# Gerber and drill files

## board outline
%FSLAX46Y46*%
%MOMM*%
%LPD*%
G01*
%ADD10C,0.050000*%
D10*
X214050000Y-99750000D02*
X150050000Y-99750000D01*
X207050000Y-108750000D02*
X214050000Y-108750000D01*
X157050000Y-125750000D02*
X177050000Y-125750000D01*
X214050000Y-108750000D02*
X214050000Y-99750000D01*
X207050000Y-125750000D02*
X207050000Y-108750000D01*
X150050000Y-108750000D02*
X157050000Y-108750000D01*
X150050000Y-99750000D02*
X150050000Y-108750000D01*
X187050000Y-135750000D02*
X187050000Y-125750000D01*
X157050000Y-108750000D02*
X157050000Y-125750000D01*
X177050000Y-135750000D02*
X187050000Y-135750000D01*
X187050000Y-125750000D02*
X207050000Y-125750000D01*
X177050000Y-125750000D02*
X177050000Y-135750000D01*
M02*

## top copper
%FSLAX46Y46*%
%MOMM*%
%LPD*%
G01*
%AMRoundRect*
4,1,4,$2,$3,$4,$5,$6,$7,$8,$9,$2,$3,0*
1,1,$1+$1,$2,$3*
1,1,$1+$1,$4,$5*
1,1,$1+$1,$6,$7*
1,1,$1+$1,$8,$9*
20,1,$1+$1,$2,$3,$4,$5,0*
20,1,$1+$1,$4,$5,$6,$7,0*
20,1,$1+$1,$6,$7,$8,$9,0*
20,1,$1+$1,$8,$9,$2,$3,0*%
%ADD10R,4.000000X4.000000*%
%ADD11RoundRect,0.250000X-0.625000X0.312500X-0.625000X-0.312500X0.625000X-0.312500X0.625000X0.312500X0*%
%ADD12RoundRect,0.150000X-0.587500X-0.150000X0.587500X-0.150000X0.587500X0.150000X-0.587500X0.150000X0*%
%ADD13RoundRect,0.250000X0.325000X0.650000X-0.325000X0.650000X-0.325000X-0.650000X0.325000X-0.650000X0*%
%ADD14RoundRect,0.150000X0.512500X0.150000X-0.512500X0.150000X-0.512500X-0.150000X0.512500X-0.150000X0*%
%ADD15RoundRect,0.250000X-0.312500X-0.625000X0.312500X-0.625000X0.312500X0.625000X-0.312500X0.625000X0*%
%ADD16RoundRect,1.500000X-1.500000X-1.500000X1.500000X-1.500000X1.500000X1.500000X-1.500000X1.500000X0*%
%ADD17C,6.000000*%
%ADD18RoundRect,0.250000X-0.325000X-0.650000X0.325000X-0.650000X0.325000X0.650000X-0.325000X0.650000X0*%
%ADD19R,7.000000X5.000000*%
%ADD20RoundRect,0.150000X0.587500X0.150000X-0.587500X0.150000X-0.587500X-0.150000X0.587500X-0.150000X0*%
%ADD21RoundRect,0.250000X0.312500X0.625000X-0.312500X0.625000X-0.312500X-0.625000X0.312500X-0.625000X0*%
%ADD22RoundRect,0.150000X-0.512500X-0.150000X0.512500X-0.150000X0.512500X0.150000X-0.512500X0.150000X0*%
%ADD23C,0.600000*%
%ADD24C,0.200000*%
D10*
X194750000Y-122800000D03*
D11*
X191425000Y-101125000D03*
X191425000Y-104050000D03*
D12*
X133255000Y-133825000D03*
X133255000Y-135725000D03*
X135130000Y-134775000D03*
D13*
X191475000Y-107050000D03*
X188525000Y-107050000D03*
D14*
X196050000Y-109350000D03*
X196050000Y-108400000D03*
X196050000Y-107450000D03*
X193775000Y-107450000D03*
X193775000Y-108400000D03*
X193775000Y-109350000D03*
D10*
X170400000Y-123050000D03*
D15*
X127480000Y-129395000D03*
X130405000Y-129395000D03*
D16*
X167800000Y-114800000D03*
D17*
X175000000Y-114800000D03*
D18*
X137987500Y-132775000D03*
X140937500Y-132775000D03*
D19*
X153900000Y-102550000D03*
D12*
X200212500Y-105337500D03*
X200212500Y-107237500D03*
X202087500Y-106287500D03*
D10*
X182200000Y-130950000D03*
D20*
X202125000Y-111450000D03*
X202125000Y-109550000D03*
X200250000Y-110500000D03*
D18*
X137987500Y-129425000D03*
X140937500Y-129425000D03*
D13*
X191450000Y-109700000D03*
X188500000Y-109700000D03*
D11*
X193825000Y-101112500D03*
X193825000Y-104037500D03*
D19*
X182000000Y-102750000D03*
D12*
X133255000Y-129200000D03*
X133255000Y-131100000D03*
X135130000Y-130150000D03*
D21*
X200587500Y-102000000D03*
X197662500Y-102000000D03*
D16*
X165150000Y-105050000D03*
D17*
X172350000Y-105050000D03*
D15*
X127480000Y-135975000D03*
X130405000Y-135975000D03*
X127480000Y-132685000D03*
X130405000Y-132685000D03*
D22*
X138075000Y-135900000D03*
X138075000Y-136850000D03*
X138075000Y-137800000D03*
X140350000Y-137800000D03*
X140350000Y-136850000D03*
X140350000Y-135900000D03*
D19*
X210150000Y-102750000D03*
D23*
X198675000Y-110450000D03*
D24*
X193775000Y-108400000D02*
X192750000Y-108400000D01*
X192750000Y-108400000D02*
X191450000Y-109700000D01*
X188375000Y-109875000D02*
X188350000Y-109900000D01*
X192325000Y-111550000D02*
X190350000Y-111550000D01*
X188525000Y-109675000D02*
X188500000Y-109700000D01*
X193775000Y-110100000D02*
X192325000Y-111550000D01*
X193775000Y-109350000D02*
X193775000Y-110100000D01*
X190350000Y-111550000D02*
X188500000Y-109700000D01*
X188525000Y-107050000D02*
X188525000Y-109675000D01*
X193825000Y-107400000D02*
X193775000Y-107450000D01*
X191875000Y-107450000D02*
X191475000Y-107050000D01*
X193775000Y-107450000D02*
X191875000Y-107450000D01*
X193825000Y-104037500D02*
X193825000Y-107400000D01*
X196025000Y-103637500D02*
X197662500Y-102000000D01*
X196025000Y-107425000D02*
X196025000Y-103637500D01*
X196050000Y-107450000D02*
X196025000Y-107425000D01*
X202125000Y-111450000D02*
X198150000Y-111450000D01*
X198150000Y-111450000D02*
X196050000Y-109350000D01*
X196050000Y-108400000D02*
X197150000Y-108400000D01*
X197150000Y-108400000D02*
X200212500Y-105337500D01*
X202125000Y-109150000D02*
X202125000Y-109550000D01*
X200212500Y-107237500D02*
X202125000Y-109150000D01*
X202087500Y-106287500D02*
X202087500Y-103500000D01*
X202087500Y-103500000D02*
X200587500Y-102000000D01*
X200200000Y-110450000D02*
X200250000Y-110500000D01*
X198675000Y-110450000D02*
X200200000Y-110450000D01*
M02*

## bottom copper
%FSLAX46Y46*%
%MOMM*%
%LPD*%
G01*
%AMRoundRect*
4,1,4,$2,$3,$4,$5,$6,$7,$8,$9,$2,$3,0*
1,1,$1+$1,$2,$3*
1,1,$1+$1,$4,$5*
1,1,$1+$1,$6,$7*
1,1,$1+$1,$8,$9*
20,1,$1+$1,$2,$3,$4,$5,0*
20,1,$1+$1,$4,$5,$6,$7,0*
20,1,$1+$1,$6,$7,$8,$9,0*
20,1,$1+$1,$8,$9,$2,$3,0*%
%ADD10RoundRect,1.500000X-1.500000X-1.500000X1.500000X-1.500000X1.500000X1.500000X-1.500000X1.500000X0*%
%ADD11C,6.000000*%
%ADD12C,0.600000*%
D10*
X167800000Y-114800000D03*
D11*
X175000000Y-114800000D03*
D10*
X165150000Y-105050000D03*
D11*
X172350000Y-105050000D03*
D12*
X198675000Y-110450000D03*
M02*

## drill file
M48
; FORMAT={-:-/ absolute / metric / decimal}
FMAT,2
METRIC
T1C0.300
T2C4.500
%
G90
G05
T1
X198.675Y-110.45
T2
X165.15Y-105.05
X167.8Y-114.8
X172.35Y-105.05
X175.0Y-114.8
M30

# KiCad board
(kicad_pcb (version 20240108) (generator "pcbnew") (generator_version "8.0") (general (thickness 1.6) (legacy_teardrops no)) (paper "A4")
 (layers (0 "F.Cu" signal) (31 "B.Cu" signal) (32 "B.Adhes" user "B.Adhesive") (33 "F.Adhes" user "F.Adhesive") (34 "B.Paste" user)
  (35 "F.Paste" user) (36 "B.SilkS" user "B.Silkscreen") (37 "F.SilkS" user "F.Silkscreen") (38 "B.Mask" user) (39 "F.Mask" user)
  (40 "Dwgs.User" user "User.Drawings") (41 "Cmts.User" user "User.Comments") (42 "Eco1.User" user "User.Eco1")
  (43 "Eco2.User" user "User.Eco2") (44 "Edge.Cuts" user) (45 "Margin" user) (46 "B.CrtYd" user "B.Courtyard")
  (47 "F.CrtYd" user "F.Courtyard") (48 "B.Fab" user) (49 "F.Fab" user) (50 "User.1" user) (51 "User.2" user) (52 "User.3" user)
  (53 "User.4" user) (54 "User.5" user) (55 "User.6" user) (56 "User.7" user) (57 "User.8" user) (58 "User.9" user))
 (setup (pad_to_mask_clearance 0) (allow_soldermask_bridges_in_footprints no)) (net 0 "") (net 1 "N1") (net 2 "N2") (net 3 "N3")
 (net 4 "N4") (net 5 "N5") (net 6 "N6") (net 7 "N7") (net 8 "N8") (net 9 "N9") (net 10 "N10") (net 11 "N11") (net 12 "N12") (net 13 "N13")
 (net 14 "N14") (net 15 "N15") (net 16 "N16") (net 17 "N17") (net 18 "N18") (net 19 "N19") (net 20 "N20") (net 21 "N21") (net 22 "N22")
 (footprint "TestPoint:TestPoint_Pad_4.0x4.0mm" (layer "F.Cu") (at 194.75 122.8)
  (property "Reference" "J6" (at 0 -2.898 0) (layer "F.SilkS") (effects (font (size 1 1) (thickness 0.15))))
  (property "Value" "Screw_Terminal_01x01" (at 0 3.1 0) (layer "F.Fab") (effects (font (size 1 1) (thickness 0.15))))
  (pad "1" smd rect (at 0 0) (size 4 4) (layers "F.Cu" "F.Mask") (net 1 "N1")))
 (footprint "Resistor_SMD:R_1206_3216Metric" (layer "F.Cu") (at 191.425 102.5875 -90)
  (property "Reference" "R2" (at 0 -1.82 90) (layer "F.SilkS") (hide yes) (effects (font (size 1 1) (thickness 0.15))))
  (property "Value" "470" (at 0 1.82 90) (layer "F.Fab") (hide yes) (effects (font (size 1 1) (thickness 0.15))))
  (pad "1" smd roundrect (at -1.4625 0 270) (size 1.125 1.75) (layers "F.Cu" "F.Paste" "F.Mask") (roundrect_rratio 0.222222) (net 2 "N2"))
  (pad "2" smd roundrect (at 1.4625 0 270) (size 1.125 1.75) (layers "F.Cu" "F.Paste" "F.Mask") (roundrect_rratio 0.222222) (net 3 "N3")))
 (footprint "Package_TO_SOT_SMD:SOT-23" (layer "F.Cu") (at 134.1925 134.775)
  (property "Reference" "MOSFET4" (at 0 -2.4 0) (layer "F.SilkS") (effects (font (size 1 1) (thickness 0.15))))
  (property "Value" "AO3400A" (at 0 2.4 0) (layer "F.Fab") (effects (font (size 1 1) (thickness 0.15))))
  (pad "1" smd roundrect (at -0.9375 -0.95) (size 1.475 0.6) (layers "F.Cu" "F.Paste" "F.Mask") (roundrect_rratio 0.25) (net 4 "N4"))
  (pad "2" smd roundrect (at -0.9375 0.95) (size 1.475 0.6) (layers "F.Cu" "F.Paste" "F.Mask") (roundrect_rratio 0.25) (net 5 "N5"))
  (pad "3" smd roundrect (at 0.9375 0) (size 1.475 0.6) (layers "F.Cu" "F.Paste" "F.Mask") (roundrect_rratio 0.25) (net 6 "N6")))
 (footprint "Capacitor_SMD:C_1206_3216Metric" (layer "F.Cu") (at 190 107.05 180)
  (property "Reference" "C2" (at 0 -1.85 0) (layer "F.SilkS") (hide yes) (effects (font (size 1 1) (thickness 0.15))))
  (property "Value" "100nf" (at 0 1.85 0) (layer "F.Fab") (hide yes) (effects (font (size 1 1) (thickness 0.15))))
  (pad "1" smd roundrect (at -1.475 0 180) (size 1.15 1.8) (layers "F.Cu" "F.Paste" "F.Mask") (roundrect_rratio 0.217391) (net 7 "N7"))
  (pad "2" smd roundrect (at 1.475 0 180) (size 1.15 1.8) (layers "F.Cu" "F.Paste" "F.Mask") (roundrect_rratio 0.217391) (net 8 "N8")))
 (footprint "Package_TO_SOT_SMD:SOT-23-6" (layer "F.Cu") (at 194.9125 108.4 180)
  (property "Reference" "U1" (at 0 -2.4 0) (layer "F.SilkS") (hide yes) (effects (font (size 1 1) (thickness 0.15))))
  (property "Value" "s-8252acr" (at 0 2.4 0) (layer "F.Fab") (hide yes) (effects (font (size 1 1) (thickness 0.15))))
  (pad "1" smd roundrect (at -1.1375 -0.95 180) (size 1.325 0.6) (layers "F.Cu" "F.Paste" "F.Mask") (roundrect_rratio 0.25) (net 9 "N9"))
  (pad "2" smd roundrect (at -1.1375 0 180) (size 1.325 0.6) (layers "F.Cu" "F.Paste" "F.Mask") (roundrect_rratio 0.25) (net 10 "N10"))
  (pad "3" smd roundrect (at -1.1375 0.95 180) (size 1.325 0.6) (layers "F.Cu" "F.Paste" "F.Mask") (roundrect_rratio 0.25) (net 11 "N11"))
  (pad "4" smd roundrect (at 1.1375 0.95 180) (size 1.325 0.6) (layers "F.Cu" "F.Paste" "F.Mask") (roundrect_rratio 0.25) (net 7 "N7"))
  (pad "5" smd roundrect (at 1.1375 0 180) (size 1.325 0.6) (layers "F.Cu" "F.Paste" "F.Mask") (roundrect_rratio 0.25) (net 3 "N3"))
  (pad "6" smd roundrect (at 1.1375 -0.95 180) (size 1.325 0.6) (layers "F.Cu" "F.Paste" "F.Mask") (roundrect_rratio 0.25) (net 8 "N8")))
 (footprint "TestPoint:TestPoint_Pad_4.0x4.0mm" (layer "F.Cu") (at 170.4 123.05)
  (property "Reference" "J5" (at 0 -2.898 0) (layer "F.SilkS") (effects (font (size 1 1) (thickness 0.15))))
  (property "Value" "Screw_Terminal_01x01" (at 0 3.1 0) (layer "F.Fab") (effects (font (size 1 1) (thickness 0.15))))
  (pad "1" smd rect (at 0 0) (size 4 4) (layers "F.Cu" "F.Mask") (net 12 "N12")))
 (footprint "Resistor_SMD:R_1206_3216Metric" (layer "F.Cu") (at 128.9425 129.395)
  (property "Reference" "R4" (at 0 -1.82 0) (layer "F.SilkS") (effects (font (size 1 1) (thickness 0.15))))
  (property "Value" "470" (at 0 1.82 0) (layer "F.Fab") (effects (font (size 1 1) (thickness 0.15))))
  (pad "1" smd roundrect (at -1.4625 0) (size 1.125 1.75) (layers "F.Cu" "F.Paste" "F.Mask") (roundrect_rratio 0.222222) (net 12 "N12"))
  (pad "2" smd roundrect (at 1.4625 0) (size 1.125 1.75) (layers "F.Cu" "F.Paste" "F.Mask") (roundrect_rratio 0.222222) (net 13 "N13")))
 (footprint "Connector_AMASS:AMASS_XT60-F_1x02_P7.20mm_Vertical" (layer "F.Cu") (at 167.8 114.8)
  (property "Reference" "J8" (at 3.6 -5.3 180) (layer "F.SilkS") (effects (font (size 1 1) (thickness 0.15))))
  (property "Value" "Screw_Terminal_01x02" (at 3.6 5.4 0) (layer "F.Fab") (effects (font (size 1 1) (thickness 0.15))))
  (pad "1" thru_hole roundrect (at 0 0) (size 6 6) (drill 4.5) (layers "*.Cu" "*.Mask") (remove_unused_layers no) (roundrect_rratio 0.25)
   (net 12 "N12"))
  (pad "2" thru_hole circle (at 7.2 0) (size 6 6) (drill 4.5) (layers "*.Cu" "*.Mask") (remove_unused_layers no) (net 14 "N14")))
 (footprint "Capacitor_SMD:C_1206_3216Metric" (layer "F.Cu") (at 139.4625 132.775)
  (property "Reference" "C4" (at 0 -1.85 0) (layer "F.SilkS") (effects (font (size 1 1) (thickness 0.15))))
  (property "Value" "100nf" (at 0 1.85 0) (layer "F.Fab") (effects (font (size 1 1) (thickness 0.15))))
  (pad "1" smd roundrect (at -1.475 0) (size 1.15 1.8) (layers "F.Cu" "F.Paste" "F.Mask") (roundrect_rratio 0.217391) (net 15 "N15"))
  (pad "2" smd roundrect (at 1.475 0) (size 1.15 1.8) (layers "F.Cu" "F.Paste" "F.Mask") (roundrect_rratio 0.217391) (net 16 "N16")))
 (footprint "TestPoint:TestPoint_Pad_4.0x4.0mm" (layer "F.Cu") (at 153.9 102.55)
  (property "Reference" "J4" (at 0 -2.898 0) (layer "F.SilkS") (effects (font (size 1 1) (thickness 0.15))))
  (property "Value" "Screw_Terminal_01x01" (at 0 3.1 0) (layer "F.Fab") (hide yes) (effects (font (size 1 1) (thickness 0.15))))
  (pad "1" smd rect (at 0 0) (size 7 5) (layers "F.Cu" "F.Mask") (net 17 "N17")))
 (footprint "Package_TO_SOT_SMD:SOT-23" (layer "F.Cu") (at 201.15 106.2875)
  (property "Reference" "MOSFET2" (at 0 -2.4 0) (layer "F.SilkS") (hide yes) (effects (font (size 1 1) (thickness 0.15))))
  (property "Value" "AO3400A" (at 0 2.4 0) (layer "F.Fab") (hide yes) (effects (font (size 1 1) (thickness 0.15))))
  (pad "1" smd roundrect (at -0.9375 -0.95) (size 1.475 0.6) (layers "F.Cu" "F.Paste" "F.Mask") (roundrect_rratio 0.25) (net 10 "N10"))
  (pad "2" smd roundrect (at -0.9375 0.95) (size 1.475 0.6) (layers "F.Cu" "F.Paste" "F.Mask") (roundrect_rratio 0.25) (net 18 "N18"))
  (pad "3" smd roundrect (at 0.9375 0) (size 1.475 0.6) (layers "F.Cu" "F.Paste" "F.Mask") (roundrect_rratio 0.25) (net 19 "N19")))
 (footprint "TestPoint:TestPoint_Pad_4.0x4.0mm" (layer "F.Cu") (at 182.2 130.95)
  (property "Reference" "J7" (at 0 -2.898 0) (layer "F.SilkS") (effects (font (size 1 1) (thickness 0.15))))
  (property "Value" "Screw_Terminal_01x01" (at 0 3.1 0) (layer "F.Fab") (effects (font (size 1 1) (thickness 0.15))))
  (pad "1" smd rect (at 0 0) (size 4 4) (layers "F.Cu" "F.Mask") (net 6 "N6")))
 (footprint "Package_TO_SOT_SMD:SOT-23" (layer "F.Cu") (at 201.1875 110.5 180)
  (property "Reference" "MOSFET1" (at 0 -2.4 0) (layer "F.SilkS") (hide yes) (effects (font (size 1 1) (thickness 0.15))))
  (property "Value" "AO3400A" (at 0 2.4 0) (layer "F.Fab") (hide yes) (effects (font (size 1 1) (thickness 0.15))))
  (pad "1" smd roundrect (at -0.9375 -0.95 180) (size 1.475 0.6) (layers "F.Cu" "F.Paste" "F.Mask") (roundrect_rratio 0.25) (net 9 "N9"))
  (pad "2" smd roundrect (at -0.9375 0.95 180) (size 1.475 0.6) (layers "F.Cu" "F.Paste" "F.Mask") (roundrect_rratio 0.25) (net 18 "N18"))
  (pad "3" smd roundrect (at 0.9375 0 180) (size 1.475 0.6) (layers "F.Cu" "F.Paste" "F.Mask") (roundrect_rratio 0.25) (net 17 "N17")))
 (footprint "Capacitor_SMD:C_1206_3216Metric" (layer "F.Cu") (at 139.4625 129.425)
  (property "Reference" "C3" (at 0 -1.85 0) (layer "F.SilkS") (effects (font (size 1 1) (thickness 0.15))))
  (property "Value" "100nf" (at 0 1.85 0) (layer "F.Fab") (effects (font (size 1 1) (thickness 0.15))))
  (pad "1" smd roundrect (at -1.475 0) (size 1.15 1.8) (layers "F.Cu" "F.Paste" "F.Mask") (roundrect_rratio 0.217391) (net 13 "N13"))
  (pad "2" smd roundrect (at 1.475 0) (size 1.15 1.8) (layers "F.Cu" "F.Paste" "F.Mask") (roundrect_rratio 0.217391) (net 16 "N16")))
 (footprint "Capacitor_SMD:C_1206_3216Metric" (layer "F.Cu") (at 189.975 109.7 180)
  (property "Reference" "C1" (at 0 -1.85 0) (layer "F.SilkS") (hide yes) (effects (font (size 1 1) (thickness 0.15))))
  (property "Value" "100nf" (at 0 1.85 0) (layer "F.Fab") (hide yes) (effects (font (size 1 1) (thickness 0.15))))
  (pad "1" smd roundrect (at -1.475 0 180) (size 1.15 1.8) (layers "F.Cu" "F.Paste" "F.Mask") (roundrect_rratio 0.217391) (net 3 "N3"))
  (pad "2" smd roundrect (at 1.475 0 180) (size 1.15 1.8) (layers "F.Cu" "F.Paste" "F.Mask") (roundrect_rratio 0.217391) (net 8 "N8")))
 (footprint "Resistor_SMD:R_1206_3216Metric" (layer "F.Cu") (at 193.825 102.575 -90)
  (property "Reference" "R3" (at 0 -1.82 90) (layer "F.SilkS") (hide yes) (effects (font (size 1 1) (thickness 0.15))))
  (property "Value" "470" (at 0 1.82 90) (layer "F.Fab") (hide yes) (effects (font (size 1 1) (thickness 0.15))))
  (pad "1" smd roundrect (at -1.4625 0 270) (size 1.125 1.75) (layers "F.Cu" "F.Paste" "F.Mask") (roundrect_rratio 0.222222) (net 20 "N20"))
  (pad "2" smd roundrect (at 1.4625 0 270) (size 1.125 1.75) (layers "F.Cu" "F.Paste" "F.Mask") (roundrect_rratio 0.222222) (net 7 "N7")))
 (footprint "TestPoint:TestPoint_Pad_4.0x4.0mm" (layer "F.Cu") (at 182 102.75)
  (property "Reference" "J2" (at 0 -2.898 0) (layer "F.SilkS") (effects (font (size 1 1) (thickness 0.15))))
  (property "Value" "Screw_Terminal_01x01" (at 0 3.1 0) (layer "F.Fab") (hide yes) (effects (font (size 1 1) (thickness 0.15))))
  (pad "1" smd rect (at 0 0) (size 7 5) (layers "F.Cu" "F.Mask") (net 20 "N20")))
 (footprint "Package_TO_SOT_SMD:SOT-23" (layer "F.Cu") (at 134.1925 130.15)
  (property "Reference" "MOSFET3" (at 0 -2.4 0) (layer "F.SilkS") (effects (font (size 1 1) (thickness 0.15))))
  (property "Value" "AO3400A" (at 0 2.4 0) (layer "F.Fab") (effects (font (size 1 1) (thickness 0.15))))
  (pad "1" smd roundrect (at -0.9375 -0.95) (size 1.475 0.6) (layers "F.Cu" "F.Paste" "F.Mask") (roundrect_rratio 0.25) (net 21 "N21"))
  (pad "2" smd roundrect (at -0.9375 0.95) (size 1.475 0.6) (layers "F.Cu" "F.Paste" "F.Mask") (roundrect_rratio 0.25) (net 5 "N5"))
  (pad "3" smd roundrect (at 0.9375 0) (size 1.475 0.6) (layers "F.Cu" "F.Paste" "F.Mask") (roundrect_rratio 0.25) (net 14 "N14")))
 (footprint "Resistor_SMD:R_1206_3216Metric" (layer "F.Cu") (at 199.125 102 180)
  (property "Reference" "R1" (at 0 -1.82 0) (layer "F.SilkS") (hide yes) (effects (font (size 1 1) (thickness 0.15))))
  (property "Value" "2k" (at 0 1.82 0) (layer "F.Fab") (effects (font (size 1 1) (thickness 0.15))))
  (pad "1" smd roundrect (at -1.4625 0 180) (size 1.125 1.75) (layers "F.Cu" "F.Paste" "F.Mask") (roundrect_rratio 0.222222) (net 19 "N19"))
  (pad "2" smd roundrect (at 1.4625 0 180) (size 1.125 1.75) (layers "F.Cu" "F.Paste" "F.Mask") (roundrect_rratio 0.222222) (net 11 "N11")))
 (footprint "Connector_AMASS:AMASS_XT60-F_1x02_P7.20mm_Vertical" (layer "F.Cu") (at 165.15 105.05)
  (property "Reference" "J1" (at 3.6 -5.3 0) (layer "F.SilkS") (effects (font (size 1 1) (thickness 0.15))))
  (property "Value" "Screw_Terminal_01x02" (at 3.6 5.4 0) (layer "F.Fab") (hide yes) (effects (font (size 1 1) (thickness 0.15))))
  (pad "1" thru_hole roundrect (at 0 0) (size 6 6) (drill 4.5) (layers "*.Cu" "*.Mask") (remove_unused_layers no) (roundrect_rratio 0.25)
   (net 2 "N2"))
  (pad "2" thru_hole circle (at 7.2 0) (size 6 6) (drill 4.5) (layers "*.Cu" "*.Mask") (remove_unused_layers no) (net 19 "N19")))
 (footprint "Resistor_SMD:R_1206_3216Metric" (layer "F.Cu") (at 128.9425 135.975)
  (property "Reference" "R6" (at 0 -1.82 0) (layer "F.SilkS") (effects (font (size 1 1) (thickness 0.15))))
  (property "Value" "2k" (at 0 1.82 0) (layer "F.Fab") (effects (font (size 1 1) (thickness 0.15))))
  (pad "1" smd roundrect (at -1.4625 0) (size 1.125 1.75) (layers "F.Cu" "F.Paste" "F.Mask") (roundrect_rratio 0.222222) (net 14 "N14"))
  (pad "2" smd roundrect (at 1.4625 0) (size 1.125 1.75) (layers "F.Cu" "F.Paste" "F.Mask") (roundrect_rratio 0.222222) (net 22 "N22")))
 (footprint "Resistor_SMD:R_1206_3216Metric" (layer "F.Cu") (at 128.9425 132.685)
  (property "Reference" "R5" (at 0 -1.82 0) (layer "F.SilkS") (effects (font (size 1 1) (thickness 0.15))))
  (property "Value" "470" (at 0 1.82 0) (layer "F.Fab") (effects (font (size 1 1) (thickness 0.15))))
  (pad "1" smd roundrect (at -1.4625 0) (size 1.125 1.75) (layers "F.Cu" "F.Paste" "F.Mask") (roundrect_rratio 0.222222) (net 1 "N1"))
  (pad "2" smd roundrect (at 1.4625 0) (size 1.125 1.75) (layers "F.Cu" "F.Paste" "F.Mask") (roundrect_rratio 0.222222) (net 15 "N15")))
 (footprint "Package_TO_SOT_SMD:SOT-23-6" (layer "F.Cu") (at 139.2125 136.85)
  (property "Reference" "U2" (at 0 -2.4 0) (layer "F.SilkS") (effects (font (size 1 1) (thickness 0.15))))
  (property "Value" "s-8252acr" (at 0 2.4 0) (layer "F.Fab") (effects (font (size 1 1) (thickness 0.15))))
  (pad "1" smd roundrect (at -1.1375 -0.95) (size 1.325 0.6) (layers "F.Cu" "F.Paste" "F.Mask") (roundrect_rratio 0.25) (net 4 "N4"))
  (pad "2" smd roundrect (at -1.1375 0) (size 1.325 0.6) (layers "F.Cu" "F.Paste" "F.Mask") (roundrect_rratio 0.25) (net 21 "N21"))
  (pad "3" smd roundrect (at -1.1375 0.95) (size 1.325 0.6) (layers "F.Cu" "F.Paste" "F.Mask") (roundrect_rratio 0.25) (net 22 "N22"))
  (pad "4" smd roundrect (at 1.1375 0.95) (size 1.325 0.6) (layers "F.Cu" "F.Paste" "F.Mask") (roundrect_rratio 0.25) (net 15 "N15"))
  (pad "5" smd roundrect (at 1.1375 0) (size 1.325 0.6) (layers "F.Cu" "F.Paste" "F.Mask") (roundrect_rratio 0.25) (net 13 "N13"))
  (pad "6" smd roundrect (at 1.1375 -0.95) (size 1.325 0.6) (layers "F.Cu" "F.Paste" "F.Mask") (roundrect_rratio 0.25) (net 16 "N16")))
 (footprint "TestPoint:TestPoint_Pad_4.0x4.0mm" (layer "F.Cu") (at 210.15 102.75)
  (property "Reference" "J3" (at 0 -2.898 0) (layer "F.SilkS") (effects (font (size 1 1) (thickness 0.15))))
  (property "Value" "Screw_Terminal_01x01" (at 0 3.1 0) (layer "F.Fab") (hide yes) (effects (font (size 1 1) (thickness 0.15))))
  (pad "1" smd rect (at 0 0) (size 7 5) (layers "F.Cu" "F.Mask") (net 2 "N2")))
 (gr_line (start 214.05 99.75) (end 150.05 99.75) (stroke (width 0.05) (type default)) (layer "Edge.Cuts"))
 (gr_line (start 207.05 108.75) (end 214.05 108.75) (stroke (width 0.05) (type default)) (layer "Edge.Cuts"))
 (gr_line (start 157.05 125.75) (end 177.05 125.75) (stroke (width 0.05) (type default)) (layer "Edge.Cuts"))
 (gr_line (start 214.05 108.75) (end 214.05 99.75) (stroke (width 0.05) (type default)) (layer "Edge.Cuts"))
 (gr_line (start 207.05 125.75) (end 207.05 108.75) (stroke (width 0.05) (type default)) (layer "Edge.Cuts"))
 (gr_line (start 150.05 108.75) (end 157.05 108.75) (stroke (width 0.05) (type default)) (layer "Edge.Cuts"))
 (gr_line (start 150.05 99.75) (end 150.05 108.75) (stroke (width 0.05) (type default)) (layer "Edge.Cuts"))
 (gr_line (start 187.05 135.75) (end 187.05 125.75) (stroke (width 0.05) (type default)) (layer "Edge.Cuts"))
 (gr_line (start 157.05 108.75) (end 157.05 125.75) (stroke (width 0.05) (type default)) (layer "Edge.Cuts"))
 (gr_line (start 177.05 135.75) (end 187.05 135.75) (stroke (width 0.05) (type default)) (layer "Edge.Cuts"))
 (gr_line (start 187.05 125.75) (end 207.05 125.75) (stroke (width 0.05) (type default)) (layer "Edge.Cuts"))
 (gr_line (start 177.05 125.75) (end 177.05 135.75) (stroke (width 0.05) (type default)) (layer "Edge.Cuts"))
 (segment (start 193.775 108.4) (end 192.75 108.4) (width 0.2) (layer "F.Cu") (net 3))
 (segment (start 192.75 108.4) (end 191.45 109.7) (width 0.2) (layer "F.Cu") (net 3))
 (segment (start 188.375 109.875) (end 188.35 109.9) (width 0.2) (layer "F.Cu") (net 8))
 (segment (start 192.325 111.55) (end 190.35 111.55) (width 0.2) (layer "F.Cu") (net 8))
 (segment (start 188.525 109.675) (end 188.5 109.7) (width 0.2) (layer "F.Cu") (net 8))
 (segment (start 193.775 110.1) (end 192.325 111.55) (width 0.2) (layer "F.Cu") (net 8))
 (segment (start 193.775 109.35) (end 193.775 110.1) (width 0.2) (layer "F.Cu") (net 8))
 (segment (start 190.35 111.55) (end 188.5 109.7) (width 0.2) (layer "F.Cu") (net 8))
 (segment (start 188.525 107.05) (end 188.525 109.675) (width 0.2) (layer "F.Cu") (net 8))
 (segment (start 193.825 107.4) (end 193.775 107.45) (width 0.2) (layer "F.Cu") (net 7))
 (segment (start 191.875 107.45) (end 191.475 107.05) (width 0.2) (layer "F.Cu") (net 7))
 (segment (start 193.775 107.45) (end 191.875 107.45) (width 0.2) (layer "F.Cu") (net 7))
 (segment (start 193.825 104.0375) (end 193.825 107.4) (width 0.2) (layer "F.Cu") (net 7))
 (segment (start 196.025 103.6375) (end 197.6625 102) (width 0.2) (layer "F.Cu") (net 11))
 (segment (start 196.025 107.425) (end 196.025 103.6375) (width 0.2) (layer "F.Cu") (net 11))
 (segment (start 196.05 107.45) (end 196.025 107.425) (width 0.2) (layer "F.Cu") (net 11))
 (segment (start 202.125 111.45) (end 198.15 111.45) (width 0.2) (layer "F.Cu") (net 9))
 (segment (start 198.15 111.45) (end 196.05 109.35) (width 0.2) (layer "F.Cu") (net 9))
 (segment (start 196.05 108.4) (end 197.15 108.4) (width 0.2) (layer "F.Cu") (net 10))
 (segment (start 197.15 108.4) (end 200.2125 105.3375) (width 0.2) (layer "F.Cu") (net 10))
 (segment (start 202.125 109.15) (end 202.125 109.55) (width 0.2) (layer "F.Cu") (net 18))
 (segment (start 200.2125 107.2375) (end 202.125 109.15) (width 0.2) (layer "F.Cu") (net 18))
 (segment (start 202.0875 106.2875) (end 202.0875 103.5) (width 0.2) (layer "F.Cu") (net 19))
 (segment (start 202.0875 103.5) (end 200.5875 102) (width 0.2) (layer "F.Cu") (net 19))
 (segment (start 200.2 110.45) (end 200.25 110.5) (width 0.2) (layer "F.Cu") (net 17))
 (segment (start 198.675 110.45) (end 200.2 110.45) (width 0.2) (layer "F.Cu") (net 17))
 (via (at 198.675 110.45) (size 0.6) (drill 0.3) (layers "F.Cu" "B.Cu") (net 17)))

